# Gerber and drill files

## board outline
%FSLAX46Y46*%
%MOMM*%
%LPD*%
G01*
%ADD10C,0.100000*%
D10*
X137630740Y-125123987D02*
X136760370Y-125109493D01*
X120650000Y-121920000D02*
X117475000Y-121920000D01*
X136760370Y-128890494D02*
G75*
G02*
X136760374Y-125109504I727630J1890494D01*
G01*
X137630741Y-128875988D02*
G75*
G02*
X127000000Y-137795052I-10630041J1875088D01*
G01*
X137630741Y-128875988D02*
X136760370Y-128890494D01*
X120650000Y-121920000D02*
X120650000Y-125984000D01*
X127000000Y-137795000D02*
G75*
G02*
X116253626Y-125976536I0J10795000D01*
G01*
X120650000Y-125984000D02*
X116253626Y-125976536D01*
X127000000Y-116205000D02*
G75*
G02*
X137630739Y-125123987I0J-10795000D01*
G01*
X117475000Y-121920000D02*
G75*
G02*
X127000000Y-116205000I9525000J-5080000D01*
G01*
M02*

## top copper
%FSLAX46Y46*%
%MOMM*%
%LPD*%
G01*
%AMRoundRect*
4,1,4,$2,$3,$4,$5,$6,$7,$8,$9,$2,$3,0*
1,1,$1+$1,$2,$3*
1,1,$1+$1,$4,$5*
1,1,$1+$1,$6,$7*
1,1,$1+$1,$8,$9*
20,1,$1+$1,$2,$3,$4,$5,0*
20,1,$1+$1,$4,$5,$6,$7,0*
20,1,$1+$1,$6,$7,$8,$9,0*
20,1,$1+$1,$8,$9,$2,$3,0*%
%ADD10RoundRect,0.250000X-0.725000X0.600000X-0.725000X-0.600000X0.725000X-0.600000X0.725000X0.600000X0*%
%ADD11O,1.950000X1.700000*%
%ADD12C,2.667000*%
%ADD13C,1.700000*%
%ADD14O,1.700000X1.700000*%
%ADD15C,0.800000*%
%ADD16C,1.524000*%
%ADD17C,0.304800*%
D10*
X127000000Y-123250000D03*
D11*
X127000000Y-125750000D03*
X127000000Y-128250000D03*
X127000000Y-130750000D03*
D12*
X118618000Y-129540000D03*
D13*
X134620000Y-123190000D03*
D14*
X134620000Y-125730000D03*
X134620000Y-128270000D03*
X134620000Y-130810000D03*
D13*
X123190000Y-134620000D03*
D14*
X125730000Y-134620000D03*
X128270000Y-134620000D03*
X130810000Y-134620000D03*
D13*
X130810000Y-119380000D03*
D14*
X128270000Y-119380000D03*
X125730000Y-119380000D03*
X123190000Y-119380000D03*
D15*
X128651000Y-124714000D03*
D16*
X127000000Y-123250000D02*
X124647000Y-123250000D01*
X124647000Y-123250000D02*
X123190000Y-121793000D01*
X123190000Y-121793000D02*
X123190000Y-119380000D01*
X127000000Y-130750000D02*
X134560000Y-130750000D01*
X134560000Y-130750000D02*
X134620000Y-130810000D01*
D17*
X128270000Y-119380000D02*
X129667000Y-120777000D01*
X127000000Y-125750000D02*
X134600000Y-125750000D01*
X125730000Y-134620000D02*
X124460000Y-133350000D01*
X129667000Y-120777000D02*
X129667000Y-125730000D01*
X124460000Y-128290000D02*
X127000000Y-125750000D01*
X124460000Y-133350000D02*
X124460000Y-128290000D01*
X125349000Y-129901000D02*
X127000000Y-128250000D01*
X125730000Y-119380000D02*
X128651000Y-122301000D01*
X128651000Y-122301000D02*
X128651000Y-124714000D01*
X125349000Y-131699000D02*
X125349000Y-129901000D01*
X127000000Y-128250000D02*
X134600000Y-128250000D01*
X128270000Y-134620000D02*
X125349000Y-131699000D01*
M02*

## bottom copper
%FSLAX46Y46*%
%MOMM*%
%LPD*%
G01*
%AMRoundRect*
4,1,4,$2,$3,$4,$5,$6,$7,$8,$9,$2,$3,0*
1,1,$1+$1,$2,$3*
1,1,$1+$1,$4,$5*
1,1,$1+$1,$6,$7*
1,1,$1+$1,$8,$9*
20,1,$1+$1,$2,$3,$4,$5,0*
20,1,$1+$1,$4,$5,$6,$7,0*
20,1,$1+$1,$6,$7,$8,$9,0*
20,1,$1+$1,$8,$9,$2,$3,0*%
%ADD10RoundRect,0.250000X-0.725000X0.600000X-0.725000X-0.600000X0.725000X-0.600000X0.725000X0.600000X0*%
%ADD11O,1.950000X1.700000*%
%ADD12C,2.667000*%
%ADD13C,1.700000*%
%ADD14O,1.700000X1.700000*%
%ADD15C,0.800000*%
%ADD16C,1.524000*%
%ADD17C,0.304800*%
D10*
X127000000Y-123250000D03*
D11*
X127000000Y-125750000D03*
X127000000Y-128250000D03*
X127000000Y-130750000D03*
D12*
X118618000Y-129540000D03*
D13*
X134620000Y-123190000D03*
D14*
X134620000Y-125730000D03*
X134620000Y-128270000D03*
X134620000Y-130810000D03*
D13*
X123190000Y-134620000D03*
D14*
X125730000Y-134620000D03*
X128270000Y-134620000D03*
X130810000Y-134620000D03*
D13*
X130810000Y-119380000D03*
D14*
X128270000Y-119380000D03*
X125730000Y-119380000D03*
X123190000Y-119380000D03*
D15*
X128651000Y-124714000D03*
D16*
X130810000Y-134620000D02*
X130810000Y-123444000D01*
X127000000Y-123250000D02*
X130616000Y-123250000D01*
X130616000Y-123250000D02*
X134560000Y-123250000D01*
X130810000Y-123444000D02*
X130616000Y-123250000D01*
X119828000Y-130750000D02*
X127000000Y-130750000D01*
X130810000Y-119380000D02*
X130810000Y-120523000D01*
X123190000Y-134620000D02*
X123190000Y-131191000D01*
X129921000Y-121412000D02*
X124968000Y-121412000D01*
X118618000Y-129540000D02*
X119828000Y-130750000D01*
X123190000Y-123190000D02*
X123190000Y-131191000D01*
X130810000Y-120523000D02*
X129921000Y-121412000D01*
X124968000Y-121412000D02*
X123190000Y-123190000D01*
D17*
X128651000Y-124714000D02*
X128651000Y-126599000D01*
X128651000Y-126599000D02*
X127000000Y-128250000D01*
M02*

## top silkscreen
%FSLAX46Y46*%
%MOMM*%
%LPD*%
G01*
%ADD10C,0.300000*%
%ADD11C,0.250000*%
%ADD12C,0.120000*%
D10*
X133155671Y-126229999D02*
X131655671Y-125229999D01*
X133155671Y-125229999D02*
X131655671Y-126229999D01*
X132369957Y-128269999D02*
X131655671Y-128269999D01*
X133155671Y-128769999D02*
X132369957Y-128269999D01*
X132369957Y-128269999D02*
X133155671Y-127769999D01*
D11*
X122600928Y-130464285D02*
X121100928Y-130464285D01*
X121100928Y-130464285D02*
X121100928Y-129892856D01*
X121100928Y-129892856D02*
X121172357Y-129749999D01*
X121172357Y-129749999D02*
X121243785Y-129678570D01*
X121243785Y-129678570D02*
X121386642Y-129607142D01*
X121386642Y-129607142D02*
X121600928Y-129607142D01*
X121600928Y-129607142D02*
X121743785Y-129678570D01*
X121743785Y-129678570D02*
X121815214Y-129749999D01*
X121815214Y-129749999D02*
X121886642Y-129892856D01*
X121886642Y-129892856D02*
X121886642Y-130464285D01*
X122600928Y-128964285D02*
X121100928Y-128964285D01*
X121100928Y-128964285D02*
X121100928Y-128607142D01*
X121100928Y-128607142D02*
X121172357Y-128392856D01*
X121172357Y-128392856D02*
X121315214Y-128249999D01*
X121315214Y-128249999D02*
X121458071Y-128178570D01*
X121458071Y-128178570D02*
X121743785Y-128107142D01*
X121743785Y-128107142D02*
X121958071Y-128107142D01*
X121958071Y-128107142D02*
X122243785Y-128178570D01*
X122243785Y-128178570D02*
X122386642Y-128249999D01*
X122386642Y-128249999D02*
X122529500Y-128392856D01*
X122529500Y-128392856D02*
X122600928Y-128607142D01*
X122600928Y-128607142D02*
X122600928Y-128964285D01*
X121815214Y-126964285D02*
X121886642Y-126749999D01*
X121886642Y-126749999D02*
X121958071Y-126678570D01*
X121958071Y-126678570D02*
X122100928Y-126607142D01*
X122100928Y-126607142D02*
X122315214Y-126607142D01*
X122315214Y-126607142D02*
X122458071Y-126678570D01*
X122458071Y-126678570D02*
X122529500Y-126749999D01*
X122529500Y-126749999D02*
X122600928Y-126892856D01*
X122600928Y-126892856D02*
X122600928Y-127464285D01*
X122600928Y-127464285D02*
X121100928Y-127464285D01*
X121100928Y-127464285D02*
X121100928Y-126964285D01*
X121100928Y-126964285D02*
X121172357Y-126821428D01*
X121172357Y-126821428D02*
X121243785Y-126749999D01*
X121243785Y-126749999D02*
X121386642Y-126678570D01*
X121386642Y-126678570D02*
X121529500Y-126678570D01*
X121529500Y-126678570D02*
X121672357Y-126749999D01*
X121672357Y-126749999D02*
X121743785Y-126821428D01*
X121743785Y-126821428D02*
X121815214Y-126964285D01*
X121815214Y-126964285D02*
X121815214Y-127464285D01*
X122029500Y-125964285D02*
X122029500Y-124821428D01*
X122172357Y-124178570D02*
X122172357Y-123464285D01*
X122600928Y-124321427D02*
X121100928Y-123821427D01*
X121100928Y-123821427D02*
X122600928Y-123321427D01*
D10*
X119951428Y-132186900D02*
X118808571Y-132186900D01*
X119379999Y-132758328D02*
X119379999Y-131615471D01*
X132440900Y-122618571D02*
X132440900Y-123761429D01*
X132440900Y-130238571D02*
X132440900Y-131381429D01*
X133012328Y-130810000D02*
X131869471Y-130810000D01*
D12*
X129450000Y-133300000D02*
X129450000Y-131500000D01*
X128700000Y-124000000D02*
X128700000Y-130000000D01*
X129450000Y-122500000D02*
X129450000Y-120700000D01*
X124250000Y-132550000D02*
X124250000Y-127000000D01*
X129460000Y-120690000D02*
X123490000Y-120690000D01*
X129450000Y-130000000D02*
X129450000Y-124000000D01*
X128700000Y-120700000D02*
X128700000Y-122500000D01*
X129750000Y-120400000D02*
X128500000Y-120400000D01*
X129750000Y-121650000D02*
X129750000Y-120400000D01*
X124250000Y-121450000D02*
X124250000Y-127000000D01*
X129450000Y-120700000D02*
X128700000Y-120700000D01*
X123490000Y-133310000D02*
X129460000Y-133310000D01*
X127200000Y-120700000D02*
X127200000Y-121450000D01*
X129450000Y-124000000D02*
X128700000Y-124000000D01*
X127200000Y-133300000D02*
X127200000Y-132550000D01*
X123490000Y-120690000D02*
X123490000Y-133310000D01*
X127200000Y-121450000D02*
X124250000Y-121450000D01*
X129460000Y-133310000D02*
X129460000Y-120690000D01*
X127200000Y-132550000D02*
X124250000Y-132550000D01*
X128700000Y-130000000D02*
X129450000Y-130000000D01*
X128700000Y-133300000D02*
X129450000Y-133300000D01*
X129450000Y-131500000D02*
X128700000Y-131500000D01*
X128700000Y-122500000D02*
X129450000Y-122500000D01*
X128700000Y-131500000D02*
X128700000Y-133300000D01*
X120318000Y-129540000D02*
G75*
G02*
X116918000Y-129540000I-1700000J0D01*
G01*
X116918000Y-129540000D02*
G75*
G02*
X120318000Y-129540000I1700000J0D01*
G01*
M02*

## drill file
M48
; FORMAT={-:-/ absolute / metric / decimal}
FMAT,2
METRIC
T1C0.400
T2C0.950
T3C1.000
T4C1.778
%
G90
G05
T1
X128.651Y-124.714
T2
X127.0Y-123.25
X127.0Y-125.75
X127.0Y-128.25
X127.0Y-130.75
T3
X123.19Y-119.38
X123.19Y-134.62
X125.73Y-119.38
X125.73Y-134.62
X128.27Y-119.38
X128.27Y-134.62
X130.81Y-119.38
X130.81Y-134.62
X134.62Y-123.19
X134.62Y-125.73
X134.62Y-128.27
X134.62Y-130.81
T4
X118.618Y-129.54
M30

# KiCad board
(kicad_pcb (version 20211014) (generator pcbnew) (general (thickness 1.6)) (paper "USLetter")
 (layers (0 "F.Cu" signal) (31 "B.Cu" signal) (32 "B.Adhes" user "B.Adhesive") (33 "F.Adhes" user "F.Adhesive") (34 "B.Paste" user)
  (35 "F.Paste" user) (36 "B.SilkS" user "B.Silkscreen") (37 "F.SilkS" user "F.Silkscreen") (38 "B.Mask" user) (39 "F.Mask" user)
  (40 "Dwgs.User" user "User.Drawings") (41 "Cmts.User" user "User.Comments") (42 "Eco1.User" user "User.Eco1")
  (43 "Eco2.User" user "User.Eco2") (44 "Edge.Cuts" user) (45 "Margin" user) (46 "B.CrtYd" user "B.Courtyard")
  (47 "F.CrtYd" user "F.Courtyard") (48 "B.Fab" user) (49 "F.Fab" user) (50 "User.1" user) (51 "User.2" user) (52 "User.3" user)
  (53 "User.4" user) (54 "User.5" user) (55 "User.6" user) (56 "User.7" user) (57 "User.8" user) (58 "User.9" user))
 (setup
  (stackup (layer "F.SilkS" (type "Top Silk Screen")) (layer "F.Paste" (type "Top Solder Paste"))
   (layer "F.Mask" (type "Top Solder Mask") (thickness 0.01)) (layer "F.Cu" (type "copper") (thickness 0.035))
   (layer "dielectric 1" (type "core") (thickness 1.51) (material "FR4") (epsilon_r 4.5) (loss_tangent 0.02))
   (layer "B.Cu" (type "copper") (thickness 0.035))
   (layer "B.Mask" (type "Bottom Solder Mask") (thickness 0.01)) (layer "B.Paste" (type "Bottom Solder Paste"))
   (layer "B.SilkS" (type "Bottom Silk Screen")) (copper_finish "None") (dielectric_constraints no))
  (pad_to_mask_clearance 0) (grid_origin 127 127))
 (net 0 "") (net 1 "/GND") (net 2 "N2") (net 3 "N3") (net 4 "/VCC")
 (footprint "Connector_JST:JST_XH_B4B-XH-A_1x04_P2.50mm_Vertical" (layer "F.Cu") (at 127 123.25 -90)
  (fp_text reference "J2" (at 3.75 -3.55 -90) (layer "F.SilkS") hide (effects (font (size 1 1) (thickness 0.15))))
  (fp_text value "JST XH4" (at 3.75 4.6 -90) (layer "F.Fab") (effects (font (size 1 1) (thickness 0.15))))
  (fp_line (start 10.05 -2.45) (end 8.25 -2.45) (layer "F.SilkS") (width 0.12))
  (fp_line (start 0.75 -1.7) (end 6.75 -1.7) (layer "F.SilkS") (width 0.12))
  (fp_line (start -0.75 -2.45) (end -2.55 -2.45) (layer "F.SilkS") (width 0.12))
  (fp_line (start 9.3 2.75) (end 3.75 2.75) (layer "F.SilkS") (width 0.12))
  (fp_line (start -2.56 -2.46) (end -2.56 3.51) (layer "F.SilkS") (width 0.12))
  (fp_line (start 6.75 -2.45) (end 0.75 -2.45) (layer "F.SilkS") (width 0.12))
  (fp_line (start -2.55 -1.7) (end -0.75 -1.7) (layer "F.SilkS") (width 0.12))
  (fp_line (start -2.85 -2.75) (end -2.85 -1.5) (layer "F.SilkS") (width 0.12))
  (fp_line (start -1.6 -2.75) (end -2.85 -2.75) (layer "F.SilkS") (width 0.12))
  (fp_line (start -1.8 2.75) (end 3.75 2.75) (layer "F.SilkS") (width 0.12))
  (fp_line (start -2.55 -2.45) (end -2.55 -1.7) (layer "F.SilkS") (width 0.12))
  (fp_line (start 10.06 3.51) (end 10.06 -2.46) (layer "F.SilkS") (width 0.12))
  (fp_line (start -2.55 -0.2) (end -1.8 -0.2) (layer "F.SilkS") (width 0.12))
  (fp_line (start 0.75 -2.45) (end 0.75 -1.7) (layer "F.SilkS") (width 0.12))
  (fp_line (start 10.05 -0.2) (end 9.3 -0.2) (layer "F.SilkS") (width 0.12))
  (fp_line (start -2.56 3.51) (end 10.06 3.51) (layer "F.SilkS") (width 0.12))
  (fp_line (start -1.8 -0.2) (end -1.8 2.75) (layer "F.SilkS") (width 0.12))
  (fp_line (start 10.06 -2.46) (end -2.56 -2.46) (layer "F.SilkS") (width 0.12))
  (fp_line (start 9.3 -0.2) (end 9.3 2.75) (layer "F.SilkS") (width 0.12))
  (fp_line (start 6.75 -1.7) (end 6.75 -2.45) (layer "F.SilkS") (width 0.12))
  (fp_line (start 10.05 -1.7) (end 10.05 -2.45) (layer "F.SilkS") (width 0.12))
  (fp_line (start 8.25 -2.45) (end 8.25 -1.7) (layer "F.SilkS") (width 0.12))
  (fp_line (start -0.75 -1.7) (end -0.75 -2.45) (layer "F.SilkS") (width 0.12))
  (fp_line (start 8.25 -1.7) (end 10.05 -1.7) (layer "F.SilkS") (width 0.12))
  (pad "1" thru_hole roundrect (at 0 0 270) (size 1.7 1.95) (drill 0.95) (layers *.Cu *.Mask) (roundrect_rratio 0.1470588235) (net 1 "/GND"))
  (pad "2" thru_hole oval (at 2.5 0 270) (size 1.7 1.95) (drill 0.95) (layers *.Cu *.Mask) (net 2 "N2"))
  (pad "3" thru_hole oval (at 5 0 270) (size 1.7 1.95) (drill 0.95) (layers *.Cu *.Mask) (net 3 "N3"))
  (pad "4" thru_hole oval (at 7.5 0 270) (size 1.7 1.95) (drill 0.95) (layers *.Cu *.Mask) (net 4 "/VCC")))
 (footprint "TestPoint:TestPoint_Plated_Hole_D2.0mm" (layer "F.Cu") (at 118.618 129.54)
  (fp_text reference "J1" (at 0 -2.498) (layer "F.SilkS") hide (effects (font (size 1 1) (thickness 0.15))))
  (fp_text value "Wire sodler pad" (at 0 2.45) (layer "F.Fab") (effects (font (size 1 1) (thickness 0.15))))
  (fp_circle (center 0 0) (end 0 -1.7) (layer "F.SilkS") (width 0.12) (fill none))
  (pad "1" thru_hole circle (at 0 0) (size 2.667 2.667) (drill 1.778) (layers *.Cu *.Mask) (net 4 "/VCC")))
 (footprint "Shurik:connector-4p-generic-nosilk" (layer "F.Cu") (at 134.62 123.19)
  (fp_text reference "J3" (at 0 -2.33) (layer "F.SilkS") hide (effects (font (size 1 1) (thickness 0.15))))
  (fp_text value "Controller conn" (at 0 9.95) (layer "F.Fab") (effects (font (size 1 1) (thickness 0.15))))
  (pad "1" thru_hole circle (at 0 0) (size 1.7 1.7) (drill 1) (layers *.Cu *.Mask) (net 1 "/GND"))
  (pad "2" thru_hole oval (at 0 2.54) (size 1.7 1.7) (drill 1) (layers *.Cu *.Mask) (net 2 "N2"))
  (pad "3" thru_hole oval (at 0 5.08) (size 1.7 1.7) (drill 1) (layers *.Cu *.Mask) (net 3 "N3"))
  (pad "4" thru_hole oval (at 0 7.62) (size 1.7 1.7) (drill 1) (layers *.Cu *.Mask) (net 4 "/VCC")))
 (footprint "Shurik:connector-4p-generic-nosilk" (layer "F.Cu") (at 123.19 134.62 90)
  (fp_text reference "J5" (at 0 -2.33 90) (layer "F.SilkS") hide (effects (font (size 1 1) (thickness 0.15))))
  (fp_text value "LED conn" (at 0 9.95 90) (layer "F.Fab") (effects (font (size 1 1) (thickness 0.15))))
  (pad "1" thru_hole circle (at 0 0 90) (size 1.7 1.7) (drill 1) (layers *.Cu *.Mask) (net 4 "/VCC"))
  (pad "2" thru_hole oval (at 0 2.54 90) (size 1.7 1.7) (drill 1) (layers *.Cu *.Mask) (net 2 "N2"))
  (pad "3" thru_hole oval (at 0 5.08 90) (size 1.7 1.7) (drill 1) (layers *.Cu *.Mask) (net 3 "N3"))
  (pad "4" thru_hole oval (at 0 7.62 90) (size 1.7 1.7) (drill 1) (layers *.Cu *.Mask) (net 1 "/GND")))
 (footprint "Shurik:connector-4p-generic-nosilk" (layer "F.Cu") (at 130.81 119.38 -90)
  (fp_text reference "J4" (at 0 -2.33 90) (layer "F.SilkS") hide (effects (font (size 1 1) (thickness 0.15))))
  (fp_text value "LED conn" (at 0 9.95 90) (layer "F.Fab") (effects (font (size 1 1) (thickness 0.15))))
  (pad "1" thru_hole circle (at 0 0 270) (size 1.7 1.7) (drill 1) (layers *.Cu *.Mask) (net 4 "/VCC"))
  (pad "2" thru_hole oval (at 0 2.54 270) (size 1.7 1.7) (drill 1) (layers *.Cu *.Mask) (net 2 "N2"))
  (pad "3" thru_hole oval (at 0 5.08 270) (size 1.7 1.7) (drill 1) (layers *.Cu *.Mask) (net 3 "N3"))
  (pad "4" thru_hole oval (at 0 7.62 270) (size 1.7 1.7) (drill 1) (layers *.Cu *.Mask) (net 1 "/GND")))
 (gr_line (start 137.63074 125.123987) (end 136.76037 125.109493) (layer "Edge.Cuts") (width 0.1))
 (gr_line (start 120.65 121.92) (end 117.475 121.92) (layer "Edge.Cuts") (width 0.1))
 (gr_arc (start 136.76037 128.890494) (mid 135.462276 126.999993) (end 136.76037 125.109493) (layer "Edge.Cuts") (width 0.1))
 (gr_arc (start 137.630741 128.875988) (mid 133.938498 135.27013) (end 127 137.795) (layer "Edge.Cuts") (width 0.1))
 (gr_line (start 137.630741 128.875988) (end 136.76037 128.890494) (layer "Edge.Cuts") (width 0.1))
 (gr_line (start 120.65 121.92) (end 120.65 125.984) (layer "Edge.Cuts") (width 0.1))
 (gr_arc (start 127 137.795) (mid 119.013129 134.262356) (end 116.253626 125.976536) (layer "Edge.Cuts") (width 0.1))
 (gr_line (start 120.65 125.984) (end 116.253626 125.976536) (layer "Edge.Cuts") (width 0.1))
 (gr_arc (start 127 116.205) (mid 133.93832 118.730063) (end 137.63074 125.123987) (layer "Edge.Cuts") (width 0.1))
 (gr_arc (start 117.475 121.92) (mid 121.446017 117.743361) (end 127 116.205) (layer "Edge.Cuts") (width 0.1))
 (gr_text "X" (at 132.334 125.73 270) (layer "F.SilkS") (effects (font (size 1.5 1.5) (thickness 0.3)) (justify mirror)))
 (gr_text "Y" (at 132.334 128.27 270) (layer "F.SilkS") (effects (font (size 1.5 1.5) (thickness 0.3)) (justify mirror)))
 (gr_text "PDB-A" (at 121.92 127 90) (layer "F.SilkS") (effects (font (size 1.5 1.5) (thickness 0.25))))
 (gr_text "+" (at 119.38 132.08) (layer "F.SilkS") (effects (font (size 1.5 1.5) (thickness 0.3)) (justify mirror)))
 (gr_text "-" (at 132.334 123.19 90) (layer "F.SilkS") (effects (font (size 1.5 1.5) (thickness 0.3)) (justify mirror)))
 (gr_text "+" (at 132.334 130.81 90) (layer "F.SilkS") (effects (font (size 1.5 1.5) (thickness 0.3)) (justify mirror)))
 (segment (start 127 123.25) (end 124.647 123.25) (width 1.524) (layer "F.Cu") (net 1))
 (segment (start 124.647 123.25) (end 123.19 121.793) (width 1.524) (layer "F.Cu") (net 1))
 (segment (start 123.19 121.793) (end 123.19 119.38) (width 1.524) (layer "F.Cu") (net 1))
 (segment (start 130.81 134.62) (end 130.81 123.444) (width 1.524) (layer "B.Cu") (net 1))
 (segment (start 127 123.25) (end 130.616 123.25) (width 1.524) (layer "B.Cu") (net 1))
 (segment (start 130.616 123.25) (end 134.56 123.25) (width 1.524) (layer "B.Cu") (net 1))
 (segment (start 130.81 123.444) (end 130.616 123.25) (width 1.524) (layer "B.Cu") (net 1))
 (segment (start 127 130.75) (end 134.56 130.75) (width 1.524) (layer "F.Cu") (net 4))
 (segment (start 134.56 130.75) (end 134.62 130.81) (width 1.524) (layer "F.Cu") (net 4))
 (segment (start 119.828 130.75) (end 127 130.75) (width 1.524) (layer "B.Cu") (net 4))
 (segment (start 130.81 119.38) (end 130.81 120.523) (width 1.524) (layer "B.Cu") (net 4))
 (segment (start 123.19 134.62) (end 123.19 131.191) (width 1.524) (layer "B.Cu") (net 4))
 (segment (start 129.921 121.412) (end 124.968 121.412) (width 1.524) (layer "B.Cu") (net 4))
 (segment (start 118.618 129.54) (end 119.828 130.75) (width 1.524) (layer "B.Cu") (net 4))
 (segment (start 123.19 123.19) (end 123.19 131.191) (width 1.524) (layer "B.Cu") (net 4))
 (segment (start 130.81 120.523) (end 129.921 121.412) (width 1.524) (layer "B.Cu") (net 4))
 (segment (start 124.968 121.412) (end 123.19 123.19) (width 1.524) (layer "B.Cu") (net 4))
 (segment (start 128.27 119.38) (end 129.667 120.777) (width 0.3048) (layer "F.Cu") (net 2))
 (segment (start 127 125.75) (end 134.6 125.75) (width 0.3048) (layer "F.Cu") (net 2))
 (segment (start 125.73 134.62) (end 124.46 133.35) (width 0.3048) (layer "F.Cu") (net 2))
 (segment (start 129.667 120.777) (end 129.667 125.73) (width 0.3048) (layer "F.Cu") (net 2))
 (segment (start 124.46 128.29) (end 127 125.75) (width 0.3048) (layer "F.Cu") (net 2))
 (segment (start 124.46 133.35) (end 124.46 128.29) (width 0.3048) (layer "F.Cu") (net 2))
 (segment (start 125.349 129.901) (end 127 128.25) (width 0.3048) (layer "F.Cu") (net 3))
 (segment (start 125.73 119.38) (end 128.651 122.301) (width 0.3048) (layer "F.Cu") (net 3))
 (segment (start 128.651 122.301) (end 128.651 124.714) (width 0.3048) (layer "F.Cu") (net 3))
 (segment (start 125.349 131.699) (end 125.349 129.901) (width 0.3048) (layer "F.Cu") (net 3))
 (segment (start 127 128.25) (end 134.6 128.25) (width 0.3048) (layer "F.Cu") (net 3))
 (segment (start 128.27 134.62) (end 125.349 131.699) (width 0.3048) (layer "F.Cu") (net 3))
 (via (at 128.651 124.714) (size 0.8) (drill 0.4) (layers "F.Cu" "B.Cu") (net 3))
 (segment (start 128.651 124.714) (end 128.651 126.599) (width 0.3048) (layer "B.Cu") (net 3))
 (segment (start 128.651 126.599) (end 127 128.25) (width 0.3048) (layer "B.Cu") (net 3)))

